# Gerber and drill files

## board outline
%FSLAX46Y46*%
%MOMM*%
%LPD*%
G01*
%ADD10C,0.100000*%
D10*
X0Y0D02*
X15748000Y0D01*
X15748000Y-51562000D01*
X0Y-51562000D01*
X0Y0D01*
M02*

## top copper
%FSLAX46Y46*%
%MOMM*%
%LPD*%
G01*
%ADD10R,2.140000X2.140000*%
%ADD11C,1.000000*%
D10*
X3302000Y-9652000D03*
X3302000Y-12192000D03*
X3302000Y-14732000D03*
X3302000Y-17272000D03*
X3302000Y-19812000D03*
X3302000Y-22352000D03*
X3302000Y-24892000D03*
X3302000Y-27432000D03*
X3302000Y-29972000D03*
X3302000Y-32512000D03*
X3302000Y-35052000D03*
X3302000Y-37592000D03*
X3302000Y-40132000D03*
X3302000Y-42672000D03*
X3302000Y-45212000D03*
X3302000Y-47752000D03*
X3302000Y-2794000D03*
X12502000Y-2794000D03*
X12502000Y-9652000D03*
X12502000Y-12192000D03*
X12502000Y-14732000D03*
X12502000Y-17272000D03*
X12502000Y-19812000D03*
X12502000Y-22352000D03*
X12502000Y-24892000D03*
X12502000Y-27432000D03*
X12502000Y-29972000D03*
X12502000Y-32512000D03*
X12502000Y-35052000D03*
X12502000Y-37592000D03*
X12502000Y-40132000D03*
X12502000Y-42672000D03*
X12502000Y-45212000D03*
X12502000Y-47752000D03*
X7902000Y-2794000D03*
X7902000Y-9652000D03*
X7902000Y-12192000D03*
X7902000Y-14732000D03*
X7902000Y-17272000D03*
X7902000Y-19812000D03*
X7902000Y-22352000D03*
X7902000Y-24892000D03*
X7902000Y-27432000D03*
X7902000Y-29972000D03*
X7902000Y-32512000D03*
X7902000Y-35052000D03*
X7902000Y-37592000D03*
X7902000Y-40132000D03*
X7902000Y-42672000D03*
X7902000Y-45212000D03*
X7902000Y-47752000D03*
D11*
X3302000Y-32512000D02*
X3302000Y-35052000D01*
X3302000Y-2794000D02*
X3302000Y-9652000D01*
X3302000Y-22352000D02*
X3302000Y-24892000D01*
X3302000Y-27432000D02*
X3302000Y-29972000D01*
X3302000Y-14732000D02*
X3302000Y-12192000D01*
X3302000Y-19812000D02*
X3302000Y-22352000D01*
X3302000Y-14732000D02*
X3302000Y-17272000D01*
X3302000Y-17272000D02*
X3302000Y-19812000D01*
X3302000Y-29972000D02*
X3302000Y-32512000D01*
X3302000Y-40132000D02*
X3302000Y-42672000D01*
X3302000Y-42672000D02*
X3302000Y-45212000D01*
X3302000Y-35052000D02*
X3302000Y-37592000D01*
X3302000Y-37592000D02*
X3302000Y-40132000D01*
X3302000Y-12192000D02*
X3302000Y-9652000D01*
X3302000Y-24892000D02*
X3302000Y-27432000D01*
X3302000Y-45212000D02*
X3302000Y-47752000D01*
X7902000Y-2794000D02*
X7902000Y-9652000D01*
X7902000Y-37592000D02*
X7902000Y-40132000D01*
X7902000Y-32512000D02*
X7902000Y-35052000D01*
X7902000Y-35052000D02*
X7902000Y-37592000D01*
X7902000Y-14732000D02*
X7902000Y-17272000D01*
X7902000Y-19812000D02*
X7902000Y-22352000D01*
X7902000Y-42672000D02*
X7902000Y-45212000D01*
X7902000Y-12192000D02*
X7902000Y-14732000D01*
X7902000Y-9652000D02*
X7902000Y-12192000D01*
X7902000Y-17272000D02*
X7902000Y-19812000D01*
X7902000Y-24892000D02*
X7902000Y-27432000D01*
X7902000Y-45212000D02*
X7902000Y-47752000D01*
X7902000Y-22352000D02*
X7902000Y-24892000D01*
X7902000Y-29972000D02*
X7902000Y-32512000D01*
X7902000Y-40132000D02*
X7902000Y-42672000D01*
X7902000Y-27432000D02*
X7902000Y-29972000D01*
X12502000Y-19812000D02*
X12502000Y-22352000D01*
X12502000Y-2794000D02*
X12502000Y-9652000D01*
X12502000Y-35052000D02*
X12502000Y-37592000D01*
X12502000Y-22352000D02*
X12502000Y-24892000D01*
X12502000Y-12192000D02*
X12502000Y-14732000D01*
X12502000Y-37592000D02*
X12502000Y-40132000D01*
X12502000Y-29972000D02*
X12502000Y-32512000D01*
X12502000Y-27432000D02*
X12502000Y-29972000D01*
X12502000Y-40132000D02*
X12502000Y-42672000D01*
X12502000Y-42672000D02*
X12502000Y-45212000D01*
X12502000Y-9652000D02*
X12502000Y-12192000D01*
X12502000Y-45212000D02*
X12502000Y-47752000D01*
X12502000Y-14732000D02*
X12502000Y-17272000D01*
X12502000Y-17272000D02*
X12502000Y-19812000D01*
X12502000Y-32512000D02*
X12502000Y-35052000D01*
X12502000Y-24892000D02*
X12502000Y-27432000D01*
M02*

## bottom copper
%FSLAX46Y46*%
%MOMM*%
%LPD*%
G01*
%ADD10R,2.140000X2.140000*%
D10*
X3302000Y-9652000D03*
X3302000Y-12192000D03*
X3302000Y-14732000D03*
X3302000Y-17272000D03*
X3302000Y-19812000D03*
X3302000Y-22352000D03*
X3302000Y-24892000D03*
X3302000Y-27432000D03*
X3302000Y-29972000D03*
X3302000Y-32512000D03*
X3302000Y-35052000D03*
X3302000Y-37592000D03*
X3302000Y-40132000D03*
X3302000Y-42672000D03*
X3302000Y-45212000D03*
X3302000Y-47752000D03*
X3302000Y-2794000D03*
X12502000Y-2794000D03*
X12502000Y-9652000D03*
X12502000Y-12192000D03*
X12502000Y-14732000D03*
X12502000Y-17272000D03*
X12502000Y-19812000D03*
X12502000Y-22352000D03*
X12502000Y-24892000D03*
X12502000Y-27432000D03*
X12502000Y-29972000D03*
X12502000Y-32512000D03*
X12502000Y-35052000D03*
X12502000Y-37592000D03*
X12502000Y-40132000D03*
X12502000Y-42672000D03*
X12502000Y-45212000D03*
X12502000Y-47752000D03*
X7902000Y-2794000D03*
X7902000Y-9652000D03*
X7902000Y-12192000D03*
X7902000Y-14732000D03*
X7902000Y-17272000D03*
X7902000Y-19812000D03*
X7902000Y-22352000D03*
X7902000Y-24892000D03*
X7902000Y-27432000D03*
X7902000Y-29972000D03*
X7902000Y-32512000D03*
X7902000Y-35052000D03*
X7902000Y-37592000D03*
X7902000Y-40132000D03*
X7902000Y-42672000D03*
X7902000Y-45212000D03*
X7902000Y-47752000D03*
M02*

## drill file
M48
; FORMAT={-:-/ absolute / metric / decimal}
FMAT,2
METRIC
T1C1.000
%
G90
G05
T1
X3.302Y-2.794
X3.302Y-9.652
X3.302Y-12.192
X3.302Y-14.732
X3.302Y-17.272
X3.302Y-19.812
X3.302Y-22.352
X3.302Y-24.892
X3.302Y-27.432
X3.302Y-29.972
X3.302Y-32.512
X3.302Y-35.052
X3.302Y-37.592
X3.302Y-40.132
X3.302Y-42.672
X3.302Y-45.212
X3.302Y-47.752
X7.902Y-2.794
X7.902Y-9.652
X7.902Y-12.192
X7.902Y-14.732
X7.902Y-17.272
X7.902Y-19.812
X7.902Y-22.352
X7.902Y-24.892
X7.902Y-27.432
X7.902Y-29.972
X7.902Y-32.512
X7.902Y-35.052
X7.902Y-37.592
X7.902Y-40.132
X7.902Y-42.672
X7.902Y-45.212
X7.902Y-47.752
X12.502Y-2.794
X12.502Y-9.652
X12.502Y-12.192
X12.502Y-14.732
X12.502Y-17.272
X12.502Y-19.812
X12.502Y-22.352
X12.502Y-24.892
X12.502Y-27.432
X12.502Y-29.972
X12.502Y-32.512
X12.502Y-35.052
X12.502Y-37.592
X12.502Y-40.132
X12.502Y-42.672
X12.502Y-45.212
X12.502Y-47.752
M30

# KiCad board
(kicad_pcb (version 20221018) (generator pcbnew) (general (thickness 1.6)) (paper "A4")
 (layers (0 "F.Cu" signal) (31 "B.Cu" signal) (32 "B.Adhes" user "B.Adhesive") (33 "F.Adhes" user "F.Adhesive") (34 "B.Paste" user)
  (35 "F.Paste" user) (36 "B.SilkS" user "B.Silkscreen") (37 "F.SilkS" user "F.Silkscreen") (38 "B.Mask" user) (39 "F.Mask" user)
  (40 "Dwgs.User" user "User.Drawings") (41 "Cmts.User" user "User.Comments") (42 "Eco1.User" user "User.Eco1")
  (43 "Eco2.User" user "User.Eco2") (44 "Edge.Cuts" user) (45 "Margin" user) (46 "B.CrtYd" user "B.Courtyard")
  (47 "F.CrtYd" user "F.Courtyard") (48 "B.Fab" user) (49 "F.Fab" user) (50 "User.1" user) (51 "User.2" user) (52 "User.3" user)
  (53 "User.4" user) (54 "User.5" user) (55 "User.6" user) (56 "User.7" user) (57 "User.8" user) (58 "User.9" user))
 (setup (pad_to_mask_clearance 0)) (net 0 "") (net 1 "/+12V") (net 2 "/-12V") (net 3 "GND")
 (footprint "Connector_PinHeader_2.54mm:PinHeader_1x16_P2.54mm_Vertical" (layer "F.Cu") (at 3.302 9.652)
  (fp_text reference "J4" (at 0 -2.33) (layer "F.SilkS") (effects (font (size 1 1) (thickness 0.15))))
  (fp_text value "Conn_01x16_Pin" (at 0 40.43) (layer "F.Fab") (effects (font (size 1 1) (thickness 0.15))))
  (pad "1" thru_hole rect (at 0 0) (size 2.14 2.14) (drill 1) (layers "*.Cu" "*.Mask") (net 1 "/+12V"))
  (pad "2" thru_hole rect (at 0 2.54) (size 2.14 2.14) (drill 1) (layers "*.Cu" "*.Mask") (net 1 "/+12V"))
  (pad "3" thru_hole rect (at 0 5.08) (size 2.14 2.14) (drill 1) (layers "*.Cu" "*.Mask") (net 1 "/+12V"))
  (pad "4" thru_hole rect (at 0 7.62) (size 2.14 2.14) (drill 1) (layers "*.Cu" "*.Mask") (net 1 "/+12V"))
  (pad "5" thru_hole rect (at 0 10.16) (size 2.14 2.14) (drill 1) (layers "*.Cu" "*.Mask") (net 1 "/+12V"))
  (pad "6" thru_hole rect (at 0 12.7) (size 2.14 2.14) (drill 1) (layers "*.Cu" "*.Mask") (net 1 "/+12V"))
  (pad "7" thru_hole rect (at 0 15.24) (size 2.14 2.14) (drill 1) (layers "*.Cu" "*.Mask") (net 1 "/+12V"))
  (pad "8" thru_hole rect (at 0 17.78) (size 2.14 2.14) (drill 1) (layers "*.Cu" "*.Mask") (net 1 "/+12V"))
  (pad "9" thru_hole rect (at 0 20.32) (size 2.14 2.14) (drill 1) (layers "*.Cu" "*.Mask") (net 1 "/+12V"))
  (pad "10" thru_hole rect (at 0 22.86) (size 2.14 2.14) (drill 1) (layers "*.Cu" "*.Mask") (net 1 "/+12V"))
  (pad "11" thru_hole rect (at 0 25.4) (size 2.14 2.14) (drill 1) (layers "*.Cu" "*.Mask") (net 1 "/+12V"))
  (pad "12" thru_hole rect (at 0 27.94) (size 2.14 2.14) (drill 1) (layers "*.Cu" "*.Mask") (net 1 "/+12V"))
  (pad "13" thru_hole rect (at 0 30.48) (size 2.14 2.14) (drill 1) (layers "*.Cu" "*.Mask") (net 1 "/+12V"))
  (pad "14" thru_hole rect (at 0 33.02) (size 2.14 2.14) (drill 1) (layers "*.Cu" "*.Mask") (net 1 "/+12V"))
  (pad "15" thru_hole rect (at 0 35.56) (size 2.14 2.14) (drill 1) (layers "*.Cu" "*.Mask") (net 1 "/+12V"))
  (pad "16" thru_hole rect (at 0 38.1) (size 2.14 2.14) (drill 1) (layers "*.Cu" "*.Mask") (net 1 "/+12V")))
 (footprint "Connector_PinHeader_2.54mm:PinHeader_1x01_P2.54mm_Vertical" (layer "F.Cu") (at 3.302 2.794 180)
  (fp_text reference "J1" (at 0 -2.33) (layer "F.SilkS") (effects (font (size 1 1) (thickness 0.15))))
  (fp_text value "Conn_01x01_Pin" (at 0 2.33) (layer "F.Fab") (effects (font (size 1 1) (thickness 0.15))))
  (pad "1" thru_hole rect (at 0 0 180) (size 2.14 2.14) (drill 1) (layers "*.Cu" "*.Mask") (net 1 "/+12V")))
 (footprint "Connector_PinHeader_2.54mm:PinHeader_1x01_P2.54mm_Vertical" (layer "F.Cu") (at 12.502 2.794 180)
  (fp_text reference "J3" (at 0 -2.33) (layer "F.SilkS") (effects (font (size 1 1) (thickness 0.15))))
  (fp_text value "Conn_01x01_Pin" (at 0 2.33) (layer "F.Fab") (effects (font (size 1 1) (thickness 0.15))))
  (pad "1" thru_hole rect (at 0 0 180) (size 2.14 2.14) (drill 1) (layers "*.Cu" "*.Mask") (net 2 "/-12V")))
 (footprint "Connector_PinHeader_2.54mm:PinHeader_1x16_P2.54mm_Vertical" (layer "F.Cu") (at 12.502 9.652)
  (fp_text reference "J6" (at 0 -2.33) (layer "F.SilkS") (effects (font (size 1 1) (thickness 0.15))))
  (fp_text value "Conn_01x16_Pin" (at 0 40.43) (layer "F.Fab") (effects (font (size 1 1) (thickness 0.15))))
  (pad "1" thru_hole rect (at 0 0) (size 2.14 2.14) (drill 1) (layers "*.Cu" "*.Mask") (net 2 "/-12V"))
  (pad "2" thru_hole rect (at 0 2.54) (size 2.14 2.14) (drill 1) (layers "*.Cu" "*.Mask") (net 2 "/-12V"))
  (pad "3" thru_hole rect (at 0 5.08) (size 2.14 2.14) (drill 1) (layers "*.Cu" "*.Mask") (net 2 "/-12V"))
  (pad "4" thru_hole rect (at 0 7.62) (size 2.14 2.14) (drill 1) (layers "*.Cu" "*.Mask") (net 2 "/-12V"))
  (pad "5" thru_hole rect (at 0 10.16) (size 2.14 2.14) (drill 1) (layers "*.Cu" "*.Mask") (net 2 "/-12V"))
  (pad "6" thru_hole rect (at 0 12.7) (size 2.14 2.14) (drill 1) (layers "*.Cu" "*.Mask") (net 2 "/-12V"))
  (pad "7" thru_hole rect (at 0 15.24) (size 2.14 2.14) (drill 1) (layers "*.Cu" "*.Mask") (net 2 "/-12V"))
  (pad "8" thru_hole rect (at 0 17.78) (size 2.14 2.14) (drill 1) (layers "*.Cu" "*.Mask") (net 2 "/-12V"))
  (pad "9" thru_hole rect (at 0 20.32) (size 2.14 2.14) (drill 1) (layers "*.Cu" "*.Mask") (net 2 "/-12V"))
  (pad "10" thru_hole rect (at 0 22.86) (size 2.14 2.14) (drill 1) (layers "*.Cu" "*.Mask") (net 2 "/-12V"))
  (pad "11" thru_hole rect (at 0 25.4) (size 2.14 2.14) (drill 1) (layers "*.Cu" "*.Mask") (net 2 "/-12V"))
  (pad "12" thru_hole rect (at 0 27.94) (size 2.14 2.14) (drill 1) (layers "*.Cu" "*.Mask") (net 2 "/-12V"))
  (pad "13" thru_hole rect (at 0 30.48) (size 2.14 2.14) (drill 1) (layers "*.Cu" "*.Mask") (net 2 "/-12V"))
  (pad "14" thru_hole rect (at 0 33.02) (size 2.14 2.14) (drill 1) (layers "*.Cu" "*.Mask") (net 2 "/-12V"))
  (pad "15" thru_hole rect (at 0 35.56) (size 2.14 2.14) (drill 1) (layers "*.Cu" "*.Mask") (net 2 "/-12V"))
  (pad "16" thru_hole rect (at 0 38.1) (size 2.14 2.14) (drill 1) (layers "*.Cu" "*.Mask") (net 2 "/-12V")))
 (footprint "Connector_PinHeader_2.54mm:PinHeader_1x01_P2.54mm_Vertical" (layer "F.Cu") (at 7.902 2.794 180)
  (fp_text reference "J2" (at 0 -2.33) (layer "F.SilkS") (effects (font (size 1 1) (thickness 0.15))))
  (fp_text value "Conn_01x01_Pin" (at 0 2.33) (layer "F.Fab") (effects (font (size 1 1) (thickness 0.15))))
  (pad "1" thru_hole rect (at 0 0 180) (size 2.14 2.14) (drill 1) (layers "*.Cu" "*.Mask") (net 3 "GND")))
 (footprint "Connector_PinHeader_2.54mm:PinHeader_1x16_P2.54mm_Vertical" (layer "F.Cu") (at 7.902 9.652)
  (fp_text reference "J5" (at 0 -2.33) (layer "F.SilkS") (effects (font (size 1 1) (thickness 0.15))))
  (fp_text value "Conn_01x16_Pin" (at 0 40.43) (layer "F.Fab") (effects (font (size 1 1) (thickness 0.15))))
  (pad "1" thru_hole rect (at 0 0) (size 2.14 2.14) (drill 1) (layers "*.Cu" "*.Mask") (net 3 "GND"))
  (pad "2" thru_hole rect (at 0 2.54) (size 2.14 2.14) (drill 1) (layers "*.Cu" "*.Mask") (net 3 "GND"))
  (pad "3" thru_hole rect (at 0 5.08) (size 2.14 2.14) (drill 1) (layers "*.Cu" "*.Mask") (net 3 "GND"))
  (pad "4" thru_hole rect (at 0 7.62) (size 2.14 2.14) (drill 1) (layers "*.Cu" "*.Mask") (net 3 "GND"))
  (pad "5" thru_hole rect (at 0 10.16) (size 2.14 2.14) (drill 1) (layers "*.Cu" "*.Mask") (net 3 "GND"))
  (pad "6" thru_hole rect (at 0 12.7) (size 2.14 2.14) (drill 1) (layers "*.Cu" "*.Mask") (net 3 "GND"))
  (pad "7" thru_hole rect (at 0 15.24) (size 2.14 2.14) (drill 1) (layers "*.Cu" "*.Mask") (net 3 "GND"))
  (pad "8" thru_hole rect (at 0 17.78) (size 2.14 2.14) (drill 1) (layers "*.Cu" "*.Mask") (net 3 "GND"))
  (pad "9" thru_hole rect (at 0 20.32) (size 2.14 2.14) (drill 1) (layers "*.Cu" "*.Mask") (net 3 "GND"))
  (pad "10" thru_hole rect (at 0 22.86) (size 2.14 2.14) (drill 1) (layers "*.Cu" "*.Mask") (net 3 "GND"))
  (pad "11" thru_hole rect (at 0 25.4) (size 2.14 2.14) (drill 1) (layers "*.Cu" "*.Mask") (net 3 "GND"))
  (pad "12" thru_hole rect (at 0 27.94) (size 2.14 2.14) (drill 1) (layers "*.Cu" "*.Mask") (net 3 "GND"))
  (pad "13" thru_hole rect (at 0 30.48) (size 2.14 2.14) (drill 1) (layers "*.Cu" "*.Mask") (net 3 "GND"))
  (pad "14" thru_hole rect (at 0 33.02) (size 2.14 2.14) (drill 1) (layers "*.Cu" "*.Mask") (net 3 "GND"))
  (pad "15" thru_hole rect (at 0 35.56) (size 2.14 2.14) (drill 1) (layers "*.Cu" "*.Mask") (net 3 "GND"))
  (pad "16" thru_hole rect (at 0 38.1) (size 2.14 2.14) (drill 1) (layers "*.Cu" "*.Mask") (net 3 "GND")))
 (gr_rect (start 0 0) (end 15.748 51.562) (stroke (width 0.1) (type default)) (fill none) (layer "Edge.Cuts"))
 (segment (start 3.302 32.512) (end 3.302 35.052) (width 1) (layer "F.Cu") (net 1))
 (segment (start 3.302 2.794) (end 3.302 9.652) (width 1) (layer "F.Cu") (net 1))
 (segment (start 3.302 22.352) (end 3.302 24.892) (width 1) (layer "F.Cu") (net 1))
 (segment (start 3.302 27.432) (end 3.302 29.972) (width 1) (layer "F.Cu") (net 1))
 (segment (start 3.302 14.732) (end 3.302 12.192) (width 1) (layer "F.Cu") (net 1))
 (segment (start 3.302 19.812) (end 3.302 22.352) (width 1) (layer "F.Cu") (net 1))
 (segment (start 3.302 14.732) (end 3.302 17.272) (width 1) (layer "F.Cu") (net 1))
 (segment (start 3.302 17.272) (end 3.302 19.812) (width 1) (layer "F.Cu") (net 1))
 (segment (start 3.302 29.972) (end 3.302 32.512) (width 1) (layer "F.Cu") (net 1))
 (segment (start 3.302 40.132) (end 3.302 42.672) (width 1) (layer "F.Cu") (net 1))
 (segment (start 3.302 42.672) (end 3.302 45.212) (width 1) (layer "F.Cu") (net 1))
 (segment (start 3.302 35.052) (end 3.302 37.592) (width 1) (layer "F.Cu") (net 1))
 (segment (start 3.302 37.592) (end 3.302 40.132) (width 1) (layer "F.Cu") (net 1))
 (segment (start 3.302 12.192) (end 3.302 9.652) (width 1) (layer "F.Cu") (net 1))
 (segment (start 3.302 24.892) (end 3.302 27.432) (width 1) (layer "F.Cu") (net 1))
 (segment (start 3.302 45.212) (end 3.302 47.752) (width 1) (layer "F.Cu") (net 1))
 (segment (start 7.902 2.794) (end 7.902 9.652) (width 1) (layer "F.Cu") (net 3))
 (segment (start 7.902 37.592) (end 7.902 40.132) (width 1) (layer "F.Cu") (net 3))
 (segment (start 7.902 32.512) (end 7.902 35.052) (width 1) (layer "F.Cu") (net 3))
 (segment (start 7.902 35.052) (end 7.902 37.592) (width 1) (layer "F.Cu") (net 3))
 (segment (start 7.902 14.732) (end 7.902 17.272) (width 1) (layer "F.Cu") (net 3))
 (segment (start 7.902 19.812) (end 7.902 22.352) (width 1) (layer "F.Cu") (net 3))
 (segment (start 7.902 42.672) (end 7.902 45.212) (width 1) (layer "F.Cu") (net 3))
 (segment (start 7.902 12.192) (end 7.902 14.732) (width 1) (layer "F.Cu") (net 3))
 (segment (start 7.902 9.652) (end 7.902 12.192) (width 1) (layer "F.Cu") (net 3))
 (segment (start 7.902 17.272) (end 7.902 19.812) (width 1) (layer "F.Cu") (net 3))
 (segment (start 7.902 24.892) (end 7.902 27.432) (width 1) (layer "F.Cu") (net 3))
 (segment (start 7.902 45.212) (end 7.902 47.752) (width 1) (layer "F.Cu") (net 3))
 (segment (start 7.902 22.352) (end 7.902 24.892) (width 1) (layer "F.Cu") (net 3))
 (segment (start 7.902 29.972) (end 7.902 32.512) (width 1) (layer "F.Cu") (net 3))
 (segment (start 7.902 40.132) (end 7.902 42.672) (width 1) (layer "F.Cu") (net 3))
 (segment (start 7.902 27.432) (end 7.902 29.972) (width 1) (layer "F.Cu") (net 3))
 (segment (start 12.502 19.812) (end 12.502 22.352) (width 1) (layer "F.Cu") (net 2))
 (segment (start 12.502 2.794) (end 12.502 9.652) (width 1) (layer "F.Cu") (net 2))
 (segment (start 12.502 35.052) (end 12.502 37.592) (width 1) (layer "F.Cu") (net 2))
 (segment (start 12.502 22.352) (end 12.502 24.892) (width 1) (layer "F.Cu") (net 2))
 (segment (start 12.502 12.192) (end 12.502 14.732) (width 1) (layer "F.Cu") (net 2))
 (segment (start 12.502 37.592) (end 12.502 40.132) (width 1) (layer "F.Cu") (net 2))
 (segment (start 12.502 29.972) (end 12.502 32.512) (width 1) (layer "F.Cu") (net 2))
 (segment (start 12.502 27.432) (end 12.502 29.972) (width 1) (layer "F.Cu") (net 2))
 (segment (start 12.502 40.132) (end 12.502 42.672) (width 1) (layer "F.Cu") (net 2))
 (segment (start 12.502 42.672) (end 12.502 45.212) (width 1) (layer "F.Cu") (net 2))
 (segment (start 12.502 9.652) (end 12.502 12.192) (width 1) (layer "F.Cu") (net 2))
 (segment (start 12.502 45.212) (end 12.502 47.752) (width 1) (layer "F.Cu") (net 2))
 (segment (start 12.502 14.732) (end 12.502 17.272) (width 1) (layer "F.Cu") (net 2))
 (segment (start 12.502 17.272) (end 12.502 19.812) (width 1) (layer "F.Cu") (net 2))
 (segment (start 12.502 32.512) (end 12.502 35.052) (width 1) (layer "F.Cu") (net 2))
 (segment (start 12.502 24.892) (end 12.502 27.432) (width 1) (layer "F.Cu") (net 2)))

